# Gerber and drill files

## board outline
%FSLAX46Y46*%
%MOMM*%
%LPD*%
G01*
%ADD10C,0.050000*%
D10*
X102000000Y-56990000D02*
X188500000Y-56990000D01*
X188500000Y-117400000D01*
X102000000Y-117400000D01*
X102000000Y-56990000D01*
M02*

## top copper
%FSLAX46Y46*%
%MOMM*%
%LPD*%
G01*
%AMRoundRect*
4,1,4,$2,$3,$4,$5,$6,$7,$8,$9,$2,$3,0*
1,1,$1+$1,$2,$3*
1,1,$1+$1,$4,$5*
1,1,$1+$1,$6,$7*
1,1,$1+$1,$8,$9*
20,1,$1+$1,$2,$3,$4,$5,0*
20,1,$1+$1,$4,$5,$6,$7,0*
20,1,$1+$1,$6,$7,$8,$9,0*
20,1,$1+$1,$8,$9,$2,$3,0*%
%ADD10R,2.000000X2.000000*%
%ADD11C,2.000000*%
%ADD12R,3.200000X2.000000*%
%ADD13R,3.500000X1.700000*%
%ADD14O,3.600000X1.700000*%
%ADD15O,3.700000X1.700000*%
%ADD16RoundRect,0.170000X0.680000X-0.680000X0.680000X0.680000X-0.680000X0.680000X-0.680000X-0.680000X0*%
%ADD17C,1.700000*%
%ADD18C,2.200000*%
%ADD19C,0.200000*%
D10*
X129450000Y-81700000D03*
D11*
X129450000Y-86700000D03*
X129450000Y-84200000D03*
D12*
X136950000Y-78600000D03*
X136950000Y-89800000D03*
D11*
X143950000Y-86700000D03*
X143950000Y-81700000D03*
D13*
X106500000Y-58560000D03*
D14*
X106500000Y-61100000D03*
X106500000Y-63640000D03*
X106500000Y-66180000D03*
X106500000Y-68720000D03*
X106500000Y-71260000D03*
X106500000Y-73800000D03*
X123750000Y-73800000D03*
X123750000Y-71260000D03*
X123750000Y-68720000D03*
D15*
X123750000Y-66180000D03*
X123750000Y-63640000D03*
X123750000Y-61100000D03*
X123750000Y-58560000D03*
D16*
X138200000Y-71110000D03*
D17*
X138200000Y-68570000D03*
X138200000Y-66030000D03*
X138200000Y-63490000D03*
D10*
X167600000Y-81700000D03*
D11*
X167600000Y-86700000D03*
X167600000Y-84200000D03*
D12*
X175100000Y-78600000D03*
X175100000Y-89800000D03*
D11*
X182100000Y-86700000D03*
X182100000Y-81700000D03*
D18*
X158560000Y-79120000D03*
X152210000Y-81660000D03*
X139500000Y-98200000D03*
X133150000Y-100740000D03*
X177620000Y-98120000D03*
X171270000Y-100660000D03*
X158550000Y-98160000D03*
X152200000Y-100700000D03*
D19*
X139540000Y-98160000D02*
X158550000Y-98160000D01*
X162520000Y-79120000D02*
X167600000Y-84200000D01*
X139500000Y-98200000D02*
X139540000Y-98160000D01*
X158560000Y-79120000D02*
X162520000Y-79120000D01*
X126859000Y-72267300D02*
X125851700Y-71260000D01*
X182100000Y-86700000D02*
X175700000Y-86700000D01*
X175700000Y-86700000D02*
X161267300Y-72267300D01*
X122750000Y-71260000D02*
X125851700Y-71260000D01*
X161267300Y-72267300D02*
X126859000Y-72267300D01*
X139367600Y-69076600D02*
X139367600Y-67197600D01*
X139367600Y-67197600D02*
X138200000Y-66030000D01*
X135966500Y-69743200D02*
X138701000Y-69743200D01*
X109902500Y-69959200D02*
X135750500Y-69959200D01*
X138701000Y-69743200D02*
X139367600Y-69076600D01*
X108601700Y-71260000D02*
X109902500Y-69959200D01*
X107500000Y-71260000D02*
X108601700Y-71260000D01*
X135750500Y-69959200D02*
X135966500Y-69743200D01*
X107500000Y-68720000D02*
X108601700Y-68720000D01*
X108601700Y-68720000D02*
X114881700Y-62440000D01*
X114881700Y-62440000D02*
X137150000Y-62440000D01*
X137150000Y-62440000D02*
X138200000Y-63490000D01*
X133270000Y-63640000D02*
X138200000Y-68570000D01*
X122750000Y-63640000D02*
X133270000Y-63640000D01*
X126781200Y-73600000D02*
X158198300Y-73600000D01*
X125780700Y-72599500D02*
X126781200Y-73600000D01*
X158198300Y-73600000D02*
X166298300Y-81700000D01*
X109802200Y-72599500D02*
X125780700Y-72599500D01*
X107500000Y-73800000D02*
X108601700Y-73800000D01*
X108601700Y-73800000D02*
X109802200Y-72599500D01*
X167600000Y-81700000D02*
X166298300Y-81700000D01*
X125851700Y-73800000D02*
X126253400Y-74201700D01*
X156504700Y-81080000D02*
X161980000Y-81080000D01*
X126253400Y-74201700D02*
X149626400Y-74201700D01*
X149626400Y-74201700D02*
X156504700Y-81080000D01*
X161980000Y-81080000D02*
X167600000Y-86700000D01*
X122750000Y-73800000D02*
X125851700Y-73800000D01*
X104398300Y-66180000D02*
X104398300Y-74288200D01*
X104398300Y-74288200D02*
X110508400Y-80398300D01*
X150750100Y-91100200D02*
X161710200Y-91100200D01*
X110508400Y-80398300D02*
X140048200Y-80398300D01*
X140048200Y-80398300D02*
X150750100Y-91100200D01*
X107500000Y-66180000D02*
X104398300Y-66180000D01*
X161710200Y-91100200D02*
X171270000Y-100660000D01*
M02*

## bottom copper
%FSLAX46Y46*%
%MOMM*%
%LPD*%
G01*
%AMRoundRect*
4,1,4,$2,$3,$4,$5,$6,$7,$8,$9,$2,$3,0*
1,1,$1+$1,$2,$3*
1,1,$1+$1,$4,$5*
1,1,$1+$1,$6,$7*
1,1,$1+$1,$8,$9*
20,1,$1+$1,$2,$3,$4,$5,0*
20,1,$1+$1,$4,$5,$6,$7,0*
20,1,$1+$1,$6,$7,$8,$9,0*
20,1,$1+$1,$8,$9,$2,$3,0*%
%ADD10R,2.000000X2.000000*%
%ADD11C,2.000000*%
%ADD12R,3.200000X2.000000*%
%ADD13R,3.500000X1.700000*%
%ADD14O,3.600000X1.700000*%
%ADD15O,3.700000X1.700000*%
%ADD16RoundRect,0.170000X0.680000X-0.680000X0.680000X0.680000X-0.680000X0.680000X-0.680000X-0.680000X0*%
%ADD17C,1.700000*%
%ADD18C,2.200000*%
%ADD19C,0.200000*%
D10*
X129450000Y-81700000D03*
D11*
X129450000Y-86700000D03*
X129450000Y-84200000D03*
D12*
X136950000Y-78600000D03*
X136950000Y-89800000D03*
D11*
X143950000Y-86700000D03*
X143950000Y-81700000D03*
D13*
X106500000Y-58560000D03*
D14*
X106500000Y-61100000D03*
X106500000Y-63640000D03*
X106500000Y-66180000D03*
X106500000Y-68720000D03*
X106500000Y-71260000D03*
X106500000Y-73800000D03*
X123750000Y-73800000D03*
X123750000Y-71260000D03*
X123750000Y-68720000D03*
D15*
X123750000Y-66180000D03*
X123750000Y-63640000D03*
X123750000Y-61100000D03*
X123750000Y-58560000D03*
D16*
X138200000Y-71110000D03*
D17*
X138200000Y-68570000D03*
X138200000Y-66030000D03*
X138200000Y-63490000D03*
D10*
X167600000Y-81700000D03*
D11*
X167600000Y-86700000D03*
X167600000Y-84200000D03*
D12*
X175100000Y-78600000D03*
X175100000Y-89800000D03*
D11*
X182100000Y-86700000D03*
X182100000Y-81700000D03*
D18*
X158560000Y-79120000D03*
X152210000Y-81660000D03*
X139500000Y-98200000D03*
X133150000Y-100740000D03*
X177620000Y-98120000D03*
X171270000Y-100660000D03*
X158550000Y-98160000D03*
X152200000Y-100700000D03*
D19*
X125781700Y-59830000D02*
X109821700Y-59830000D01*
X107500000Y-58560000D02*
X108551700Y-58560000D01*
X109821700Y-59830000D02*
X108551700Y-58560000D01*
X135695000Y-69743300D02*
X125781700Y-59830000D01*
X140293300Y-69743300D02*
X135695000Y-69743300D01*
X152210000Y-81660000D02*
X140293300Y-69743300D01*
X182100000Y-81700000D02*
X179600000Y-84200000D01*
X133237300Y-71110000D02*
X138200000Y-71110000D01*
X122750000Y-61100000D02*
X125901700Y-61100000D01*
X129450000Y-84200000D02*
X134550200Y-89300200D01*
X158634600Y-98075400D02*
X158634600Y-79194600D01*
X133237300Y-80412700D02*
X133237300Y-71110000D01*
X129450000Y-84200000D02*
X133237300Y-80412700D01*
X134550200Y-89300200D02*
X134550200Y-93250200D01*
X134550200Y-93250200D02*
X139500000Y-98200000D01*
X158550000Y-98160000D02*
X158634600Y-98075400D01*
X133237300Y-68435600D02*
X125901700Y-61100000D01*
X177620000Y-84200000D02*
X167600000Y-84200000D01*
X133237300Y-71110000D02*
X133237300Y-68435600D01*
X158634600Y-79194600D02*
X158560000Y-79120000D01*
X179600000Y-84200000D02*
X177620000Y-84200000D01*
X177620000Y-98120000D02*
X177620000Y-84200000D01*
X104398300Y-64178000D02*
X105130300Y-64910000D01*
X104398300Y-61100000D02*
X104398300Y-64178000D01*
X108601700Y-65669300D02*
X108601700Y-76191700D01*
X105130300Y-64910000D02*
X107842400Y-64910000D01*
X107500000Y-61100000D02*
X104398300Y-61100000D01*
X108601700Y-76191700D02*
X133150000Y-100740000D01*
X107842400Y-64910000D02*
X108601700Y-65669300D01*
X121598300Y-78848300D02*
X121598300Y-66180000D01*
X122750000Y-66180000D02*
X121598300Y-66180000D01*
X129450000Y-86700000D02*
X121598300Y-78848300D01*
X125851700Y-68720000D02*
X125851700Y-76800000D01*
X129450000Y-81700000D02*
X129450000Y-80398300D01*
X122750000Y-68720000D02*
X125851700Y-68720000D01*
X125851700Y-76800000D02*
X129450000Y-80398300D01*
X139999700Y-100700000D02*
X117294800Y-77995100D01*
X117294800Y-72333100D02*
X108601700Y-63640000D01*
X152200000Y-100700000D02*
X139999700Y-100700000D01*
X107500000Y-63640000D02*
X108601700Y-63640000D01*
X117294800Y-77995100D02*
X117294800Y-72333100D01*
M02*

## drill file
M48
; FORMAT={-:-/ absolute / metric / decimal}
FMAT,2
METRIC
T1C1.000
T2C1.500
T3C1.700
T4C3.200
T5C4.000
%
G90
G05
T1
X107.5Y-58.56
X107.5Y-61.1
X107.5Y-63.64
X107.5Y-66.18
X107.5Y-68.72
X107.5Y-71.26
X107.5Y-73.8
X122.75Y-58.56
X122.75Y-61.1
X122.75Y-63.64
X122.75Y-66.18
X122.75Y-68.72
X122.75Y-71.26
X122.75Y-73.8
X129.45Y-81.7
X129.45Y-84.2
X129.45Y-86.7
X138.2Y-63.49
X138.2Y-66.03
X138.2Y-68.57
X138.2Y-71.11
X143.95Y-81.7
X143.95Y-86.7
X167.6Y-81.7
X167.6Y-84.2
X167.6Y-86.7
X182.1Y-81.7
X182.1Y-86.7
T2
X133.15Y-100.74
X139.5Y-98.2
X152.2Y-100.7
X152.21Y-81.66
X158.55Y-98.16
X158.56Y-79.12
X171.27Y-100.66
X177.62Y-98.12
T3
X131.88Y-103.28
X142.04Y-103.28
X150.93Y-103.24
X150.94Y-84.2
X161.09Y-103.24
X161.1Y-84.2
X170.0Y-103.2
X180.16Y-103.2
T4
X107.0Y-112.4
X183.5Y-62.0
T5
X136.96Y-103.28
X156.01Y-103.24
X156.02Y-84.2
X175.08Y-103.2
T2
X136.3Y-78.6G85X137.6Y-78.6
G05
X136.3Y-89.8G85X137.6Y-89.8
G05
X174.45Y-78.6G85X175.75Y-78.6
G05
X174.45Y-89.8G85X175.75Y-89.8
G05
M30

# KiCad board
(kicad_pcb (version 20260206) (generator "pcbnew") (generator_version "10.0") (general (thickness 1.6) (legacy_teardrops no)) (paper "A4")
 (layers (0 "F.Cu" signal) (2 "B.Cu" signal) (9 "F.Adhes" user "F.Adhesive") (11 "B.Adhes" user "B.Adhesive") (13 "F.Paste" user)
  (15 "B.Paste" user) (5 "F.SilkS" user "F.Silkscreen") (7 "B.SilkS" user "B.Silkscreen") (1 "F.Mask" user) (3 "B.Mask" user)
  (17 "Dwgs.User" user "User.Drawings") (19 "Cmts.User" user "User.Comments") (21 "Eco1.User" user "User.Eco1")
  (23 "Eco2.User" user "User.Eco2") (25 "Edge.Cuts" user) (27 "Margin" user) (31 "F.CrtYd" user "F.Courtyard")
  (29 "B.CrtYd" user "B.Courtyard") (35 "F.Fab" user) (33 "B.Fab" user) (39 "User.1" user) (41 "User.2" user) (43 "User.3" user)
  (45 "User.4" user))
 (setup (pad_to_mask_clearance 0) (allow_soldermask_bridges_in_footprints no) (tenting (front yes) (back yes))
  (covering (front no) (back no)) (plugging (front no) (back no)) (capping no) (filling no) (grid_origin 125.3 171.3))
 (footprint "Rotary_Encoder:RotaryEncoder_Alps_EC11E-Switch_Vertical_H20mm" (layer "F.Cu") (at 129.45 81.7)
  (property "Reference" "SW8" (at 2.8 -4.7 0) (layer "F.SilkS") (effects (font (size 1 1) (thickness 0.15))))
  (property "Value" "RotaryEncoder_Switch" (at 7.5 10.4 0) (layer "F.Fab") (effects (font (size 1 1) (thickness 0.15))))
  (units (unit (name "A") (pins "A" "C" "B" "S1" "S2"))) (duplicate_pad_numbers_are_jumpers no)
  (pad "A" thru_hole rect (at 0 0) (size 2 2) (drill 1) (layers "*.Cu" "*.Mask") (remove_unused_layers no) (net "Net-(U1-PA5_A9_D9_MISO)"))
  (pad "B" thru_hole circle (at 0 5) (size 2 2) (drill 1) (layers "*.Cu" "*.Mask") (remove_unused_layers no)
   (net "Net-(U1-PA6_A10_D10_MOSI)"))
  (pad "C" thru_hole circle (at 0 2.5) (size 2 2) (drill 1) (layers "*.Cu" "*.Mask") (remove_unused_layers no) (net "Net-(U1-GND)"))
  (pad "MP" thru_hole rect (at 7.5 -3.1) (size 3.2 2) (drill oval 2.8 1.5) (layers "*.Cu" "*.Mask") (remove_unused_layers no))
  (pad "MP" thru_hole rect (at 7.5 8.1) (size 3.2 2) (drill oval 2.8 1.5) (layers "*.Cu" "*.Mask") (remove_unused_layers no))
  (pad "S1" thru_hole circle (at 14.5 5) (size 2 2) (drill 1) (layers "*.Cu" "*.Mask") (remove_unused_layers no)
   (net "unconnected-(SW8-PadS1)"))
  (pad "S2" thru_hole circle (at 14.5 0) (size 2 2) (drill 1) (layers "*.Cu" "*.Mask") (remove_unused_layers no)
   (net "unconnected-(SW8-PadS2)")))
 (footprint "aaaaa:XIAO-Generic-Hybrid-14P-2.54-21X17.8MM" (layer "F.Cu") (at 115.125 66.18)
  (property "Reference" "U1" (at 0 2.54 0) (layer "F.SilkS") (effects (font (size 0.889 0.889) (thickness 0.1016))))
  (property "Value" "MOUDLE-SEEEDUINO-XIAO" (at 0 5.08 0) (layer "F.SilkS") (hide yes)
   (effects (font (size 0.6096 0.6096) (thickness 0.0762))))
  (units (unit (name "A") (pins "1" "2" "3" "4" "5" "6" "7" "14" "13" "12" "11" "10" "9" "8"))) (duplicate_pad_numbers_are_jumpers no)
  (pad "1" thru_hole rect (at -7.625 -7.62) (size 3.5 1.7) (drill 1 (offset -1 0)) (layers "*.Cu" "*.Mask") (remove_unused_layers no)
   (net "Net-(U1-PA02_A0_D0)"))
  (pad "2" thru_hole oval (at -7.625 -5.08) (size 3.6 1.7) (drill 1 (offset -1 0)) (layers "*.Cu" "*.Mask") (remove_unused_layers no)
   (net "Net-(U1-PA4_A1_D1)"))
  (pad "3" thru_hole oval (at -7.625 -2.54) (size 3.6 1.7) (drill 1 (offset -1 0)) (layers "*.Cu" "*.Mask") (remove_unused_layers no)
   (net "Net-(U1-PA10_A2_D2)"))
  (pad "4" thru_hole oval (at -7.625 0) (size 3.6 1.7) (drill 1 (offset -1 0)) (layers "*.Cu" "*.Mask") (remove_unused_layers no)
   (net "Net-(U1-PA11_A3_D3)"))
  (pad "5" thru_hole oval (at -7.625 2.54) (size 3.6 1.7) (drill 1 (offset -1 0)) (layers "*.Cu" "*.Mask") (remove_unused_layers no)
   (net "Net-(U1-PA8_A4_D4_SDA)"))
  (pad "6" thru_hole oval (at -7.625 5.08 180) (size 3.6 1.7) (drill 1 (offset 1 0)) (layers "*.Cu" "*.Mask") (remove_unused_layers no)
   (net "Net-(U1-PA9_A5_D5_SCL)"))
  (pad "7" thru_hole oval (at -7.625 7.62) (size 3.6 1.7) (drill 1 (offset -1 0)) (layers "*.Cu" "*.Mask") (remove_unused_layers no)
   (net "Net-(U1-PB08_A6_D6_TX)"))
  (pad "8" thru_hole oval (at 7.625 7.62) (size 3.6 1.7) (drill 1 (offset 1 0)) (layers "*.Cu" "*.Mask") (remove_unused_layers no)
   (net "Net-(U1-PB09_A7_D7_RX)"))
  (pad "9" thru_hole oval (at 7.625 5.08) (size 3.6 1.7) (drill 1 (offset 1 0)) (layers "*.Cu" "*.Mask") (remove_unused_layers no)
   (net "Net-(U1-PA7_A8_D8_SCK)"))
  (pad "10" thru_hole oval (at 7.625 2.54) (size 3.6 1.7) (drill 1 (offset 1 0)) (layers "*.Cu" "*.Mask") (remove_unused_layers no)
   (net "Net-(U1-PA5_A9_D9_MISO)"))
  (pad "11" thru_hole oval (at 7.625 0) (size 3.7 1.7) (drill 1 (offset 1 0)) (layers "*.Cu" "*.Mask") (remove_unused_layers no)
   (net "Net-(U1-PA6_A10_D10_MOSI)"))
  (pad "12" thru_hole oval (at 7.625 -2.54) (size 3.7 1.7) (drill 1 (offset 1 0)) (layers "*.Cu" "*.Mask") (remove_unused_layers no)
   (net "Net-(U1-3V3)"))
  (pad "13" thru_hole oval (at 7.625 -5.08) (size 3.7 1.7) (drill 1 (offset 1 0)) (layers "*.Cu" "*.Mask") (remove_unused_layers no)
   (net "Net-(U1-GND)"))
  (pad "14" thru_hole oval (at 7.625 -7.62) (size 3.7 1.7) (drill 1 (offset 1 0)) (layers "*.Cu" "*.Mask") (remove_unused_layers no)
   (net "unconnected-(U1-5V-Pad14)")))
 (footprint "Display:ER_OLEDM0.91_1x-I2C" (layer "F.Cu") (at 138.2 71.11 90)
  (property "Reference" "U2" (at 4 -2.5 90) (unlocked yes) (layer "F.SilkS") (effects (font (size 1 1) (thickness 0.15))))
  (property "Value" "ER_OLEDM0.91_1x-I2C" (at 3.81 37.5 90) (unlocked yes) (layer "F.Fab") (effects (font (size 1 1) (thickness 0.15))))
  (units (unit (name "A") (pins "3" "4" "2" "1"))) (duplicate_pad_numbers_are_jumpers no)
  (pad "1" thru_hole roundrect (at 0 0 90) (size 1.7 1.7) (drill 1) (layers "*.Cu" "*.Mask") (remove_unused_layers no)
   (roundrect_rratio 0.1) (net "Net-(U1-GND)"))
  (pad "2" thru_hole circle (at 2.54 0 90) (size 1.7 1.7) (drill 1) (layers "*.Cu" "*.Mask") (remove_unused_layers no) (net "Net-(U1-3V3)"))
  (pad "3" thru_hole circle (at 5.08 0 90) (size 1.7 1.7) (drill 1) (layers "*.Cu" "*.Mask") (remove_unused_layers no)
   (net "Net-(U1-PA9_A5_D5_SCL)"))
  (pad "4" thru_hole circle (at 7.62 0 90) (size 1.7 1.7) (drill 1) (layers "*.Cu" "*.Mask") (remove_unused_layers no)
   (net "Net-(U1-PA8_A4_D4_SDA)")))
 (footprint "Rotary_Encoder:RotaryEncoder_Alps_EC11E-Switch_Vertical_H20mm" (layer "F.Cu") (at 167.6 81.7)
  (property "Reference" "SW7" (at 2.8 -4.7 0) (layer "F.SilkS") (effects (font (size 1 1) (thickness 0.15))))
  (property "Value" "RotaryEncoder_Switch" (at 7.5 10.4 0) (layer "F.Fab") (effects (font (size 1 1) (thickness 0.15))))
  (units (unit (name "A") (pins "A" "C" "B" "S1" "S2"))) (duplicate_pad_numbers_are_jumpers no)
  (pad "A" thru_hole rect (at 0 0) (size 2 2) (drill 1) (layers "*.Cu" "*.Mask") (remove_unused_layers no) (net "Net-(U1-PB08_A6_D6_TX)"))
  (pad "B" thru_hole circle (at 0 5) (size 2 2) (drill 1) (layers "*.Cu" "*.Mask") (remove_unused_layers no) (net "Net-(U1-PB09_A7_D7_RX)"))
  (pad "C" thru_hole circle (at 0 2.5) (size 2 2) (drill 1) (layers "*.Cu" "*.Mask") (remove_unused_layers no) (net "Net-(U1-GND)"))
  (pad "MP" thru_hole rect (at 7.5 -3.1) (size 3.2 2) (drill oval 2.8 1.5) (layers "*.Cu" "*.Mask") (remove_unused_layers no))
  (pad "MP" thru_hole rect (at 7.5 8.1) (size 3.2 2) (drill oval 2.8 1.5) (layers "*.Cu" "*.Mask") (remove_unused_layers no))
  (pad "S1" thru_hole circle (at 14.5 5) (size 2 2) (drill 1) (layers "*.Cu" "*.Mask") (remove_unused_layers no)
   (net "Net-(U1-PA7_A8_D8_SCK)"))
  (pad "S2" thru_hole circle (at 14.5 0) (size 2 2) (drill 1) (layers "*.Cu" "*.Mask") (remove_unused_layers no) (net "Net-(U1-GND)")))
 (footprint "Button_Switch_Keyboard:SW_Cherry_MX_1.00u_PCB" (layer "F.Cu") (at 158.56 79.12)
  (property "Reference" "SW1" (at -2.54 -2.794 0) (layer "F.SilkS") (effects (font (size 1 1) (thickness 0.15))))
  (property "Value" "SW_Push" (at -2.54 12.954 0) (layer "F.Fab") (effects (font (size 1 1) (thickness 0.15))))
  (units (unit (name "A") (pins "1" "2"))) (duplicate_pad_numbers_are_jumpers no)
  (pad "" np_thru_hole circle (at -7.62 5.08) (size 1.7 1.7) (drill 1.7) (layers "*.Cu" "*.Mask"))
  (pad "" np_thru_hole circle (at -2.54 5.08) (size 4 4) (drill 4) (layers "*.Cu" "*.Mask"))
  (pad "" np_thru_hole circle (at 2.54 5.08) (size 1.7 1.7) (drill 1.7) (layers "*.Cu" "*.Mask"))
  (pad "1" thru_hole circle (at 0 0) (size 2.2 2.2) (drill 1.5) (layers "*.Cu" "*.Mask") (remove_unused_layers no) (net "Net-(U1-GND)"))
  (pad "2" thru_hole circle (at -6.35 2.54) (size 2.2 2.2) (drill 1.5) (layers "*.Cu" "*.Mask") (remove_unused_layers no)
   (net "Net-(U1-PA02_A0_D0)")))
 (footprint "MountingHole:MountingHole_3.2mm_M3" (layer "F.Cu") (at 183.5 62)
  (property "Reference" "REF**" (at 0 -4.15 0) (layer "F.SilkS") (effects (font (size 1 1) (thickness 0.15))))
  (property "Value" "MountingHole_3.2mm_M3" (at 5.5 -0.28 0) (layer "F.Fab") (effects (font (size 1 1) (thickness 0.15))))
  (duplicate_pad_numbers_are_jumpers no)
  (pad "" np_thru_hole circle (at 0 0) (size 3.2 3.2) (drill 3.2) (layers "*.Cu" "*.Mask")))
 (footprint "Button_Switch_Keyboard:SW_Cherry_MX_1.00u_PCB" (layer "F.Cu") (at 139.5 98.2)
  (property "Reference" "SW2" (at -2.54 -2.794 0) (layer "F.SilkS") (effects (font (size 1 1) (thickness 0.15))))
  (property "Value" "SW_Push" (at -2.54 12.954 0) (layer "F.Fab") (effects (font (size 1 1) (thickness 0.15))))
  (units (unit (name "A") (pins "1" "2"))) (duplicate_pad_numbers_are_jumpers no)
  (pad "" np_thru_hole circle (at -7.62 5.08) (size 1.7 1.7) (drill 1.7) (layers "*.Cu" "*.Mask"))
  (pad "" np_thru_hole circle (at -2.54 5.08) (size 4 4) (drill 4) (layers "*.Cu" "*.Mask"))
  (pad "" np_thru_hole circle (at 2.54 5.08) (size 1.7 1.7) (drill 1.7) (layers "*.Cu" "*.Mask"))
  (pad "1" thru_hole circle (at 0 0) (size 2.2 2.2) (drill 1.5) (layers "*.Cu" "*.Mask") (remove_unused_layers no) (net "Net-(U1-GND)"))
  (pad "2" thru_hole circle (at -6.35 2.54) (size 2.2 2.2) (drill 1.5) (layers "*.Cu" "*.Mask") (remove_unused_layers no)
   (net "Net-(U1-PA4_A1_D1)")))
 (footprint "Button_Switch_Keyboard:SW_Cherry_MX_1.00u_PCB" (layer "F.Cu") (at 177.62 98.12)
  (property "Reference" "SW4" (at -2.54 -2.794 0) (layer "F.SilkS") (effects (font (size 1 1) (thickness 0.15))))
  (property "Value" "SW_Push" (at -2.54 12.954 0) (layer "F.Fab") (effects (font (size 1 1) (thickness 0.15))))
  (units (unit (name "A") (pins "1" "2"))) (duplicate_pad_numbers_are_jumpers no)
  (pad "" np_thru_hole circle (at -7.62 5.08) (size 1.7 1.7) (drill 1.7) (layers "*.Cu" "*.Mask"))
  (pad "" np_thru_hole circle (at -2.54 5.08) (size 4 4) (drill 4) (layers "*.Cu" "*.Mask"))
  (pad "" np_thru_hole circle (at 2.54 5.08) (size 1.7 1.7) (drill 1.7) (layers "*.Cu" "*.Mask"))
  (pad "1" thru_hole circle (at 0 0) (size 2.2 2.2) (drill 1.5) (layers "*.Cu" "*.Mask") (remove_unused_layers no) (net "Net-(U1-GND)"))
  (pad "2" thru_hole circle (at -6.35 2.54) (size 2.2 2.2) (drill 1.5) (layers "*.Cu" "*.Mask") (remove_unused_layers no)
   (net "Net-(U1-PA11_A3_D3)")))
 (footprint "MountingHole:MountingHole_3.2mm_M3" (layer "F.Cu") (at 107 112.4)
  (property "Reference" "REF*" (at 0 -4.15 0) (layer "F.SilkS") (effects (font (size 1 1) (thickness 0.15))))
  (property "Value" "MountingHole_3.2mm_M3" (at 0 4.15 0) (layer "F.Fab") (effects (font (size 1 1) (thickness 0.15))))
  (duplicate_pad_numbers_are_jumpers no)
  (pad "" np_thru_hole circle (at 0 0) (size 3.2 3.2) (drill 3.2) (layers "*.Cu" "*.Mask")))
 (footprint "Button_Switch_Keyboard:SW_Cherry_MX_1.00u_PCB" (layer "F.Cu") (at 158.55 98.16)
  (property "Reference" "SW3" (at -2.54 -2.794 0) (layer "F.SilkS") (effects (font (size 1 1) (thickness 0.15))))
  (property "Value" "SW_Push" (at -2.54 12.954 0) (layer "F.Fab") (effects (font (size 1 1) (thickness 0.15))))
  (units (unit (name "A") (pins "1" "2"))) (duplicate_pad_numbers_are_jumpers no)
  (pad "" np_thru_hole circle (at -7.62 5.08) (size 1.7 1.7) (drill 1.7) (layers "*.Cu" "*.Mask"))
  (pad "" np_thru_hole circle (at -2.54 5.08) (size 4 4) (drill 4) (layers "*.Cu" "*.Mask"))
  (pad "" np_thru_hole circle (at 2.54 5.08) (size 1.7 1.7) (drill 1.7) (layers "*.Cu" "*.Mask"))
  (pad "1" thru_hole circle (at 0 0) (size 2.2 2.2) (drill 1.5) (layers "*.Cu" "*.Mask") (remove_unused_layers no) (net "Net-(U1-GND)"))
  (pad "2" thru_hole circle (at -6.35 2.54) (size 2.2 2.2) (drill 1.5) (layers "*.Cu" "*.Mask") (remove_unused_layers no)
   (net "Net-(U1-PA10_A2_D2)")))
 (gr_rect (start 102 56.99) (end 188.5 117.4) (stroke (width 0.05) (type default)) (fill no) (layer "Edge.Cuts"))
 (segment (start 125.7817 59.83) (end 109.8217 59.83) (width 0.2) (layer "B.Cu") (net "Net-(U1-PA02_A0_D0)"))
 (segment (start 107.5 58.56) (end 108.5517 58.56) (width 0.2) (layer "B.Cu") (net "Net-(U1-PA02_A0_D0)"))
 (segment (start 109.8217 59.83) (end 108.5517 58.56) (width 0.2) (layer "B.Cu") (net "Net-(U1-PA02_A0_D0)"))
 (segment (start 135.695 69.7433) (end 125.7817 59.83) (width 0.2) (layer "B.Cu") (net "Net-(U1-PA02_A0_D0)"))
 (segment (start 140.2933 69.7433) (end 135.695 69.7433) (width 0.2) (layer "B.Cu") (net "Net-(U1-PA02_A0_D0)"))
 (segment (start 152.21 81.66) (end 140.2933 69.7433) (width 0.2) (layer "B.Cu") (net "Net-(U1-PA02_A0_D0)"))
 (segment (start 139.54 98.16) (end 158.55 98.16) (width 0.2) (layer "F.Cu") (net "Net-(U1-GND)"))
 (segment (start 162.52 79.12) (end 167.6 84.2) (width 0.2) (layer "F.Cu") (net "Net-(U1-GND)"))
 (segment (start 139.5 98.2) (end 139.54 98.16) (width 0.2) (layer "F.Cu") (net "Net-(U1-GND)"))
 (segment (start 158.56 79.12) (end 162.52 79.12) (width 0.2) (layer "F.Cu") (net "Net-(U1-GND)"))
 (segment (start 182.1 81.7) (end 179.6 84.2) (width 0.2) (layer "B.Cu") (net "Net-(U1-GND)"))
 (segment (start 133.2373 71.11) (end 138.2 71.11) (width 0.2) (layer "B.Cu") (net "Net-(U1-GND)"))
 (segment (start 122.75 61.1) (end 125.9017 61.1) (width 0.2) (layer "B.Cu") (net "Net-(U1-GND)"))
 (segment (start 129.45 84.2) (end 134.5502 89.3002) (width 0.2) (layer "B.Cu") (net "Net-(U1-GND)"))
 (segment (start 158.6346 98.0754) (end 158.6346 79.1946) (width 0.2) (layer "B.Cu") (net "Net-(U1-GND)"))
 (segment (start 133.2373 80.4127) (end 133.2373 71.11) (width 0.2) (layer "B.Cu") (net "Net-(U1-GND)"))
 (segment (start 129.45 84.2) (end 133.2373 80.4127) (width 0.2) (layer "B.Cu") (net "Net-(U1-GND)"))
 (segment (start 134.5502 89.3002) (end 134.5502 93.2502) (width 0.2) (layer "B.Cu") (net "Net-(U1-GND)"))
 (segment (start 134.5502 93.2502) (end 139.5 98.2) (width 0.2) (layer "B.Cu") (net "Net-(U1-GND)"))
 (segment (start 158.55 98.16) (end 158.6346 98.0754) (width 0.2) (layer "B.Cu") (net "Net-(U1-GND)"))
 (segment (start 133.2373 68.4356) (end 125.9017 61.1) (width 0.2) (layer "B.Cu") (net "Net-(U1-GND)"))
 (segment (start 177.62 84.2) (end 167.6 84.2) (width 0.2) (layer "B.Cu") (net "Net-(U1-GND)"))
 (segment (start 133.2373 71.11) (end 133.2373 68.4356) (width 0.2) (layer "B.Cu") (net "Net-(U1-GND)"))
 (segment (start 158.6346 79.1946) (end 158.56 79.12) (width 0.2) (layer "B.Cu") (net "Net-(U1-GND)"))
 (segment (start 179.6 84.2) (end 177.62 84.2) (width 0.2) (layer "B.Cu") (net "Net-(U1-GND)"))
 (segment (start 177.62 98.12) (end 177.62 84.2) (width 0.2) (layer "B.Cu") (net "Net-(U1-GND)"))
 (segment (start 104.3983 64.178) (end 105.1303 64.91) (width 0.2) (layer "B.Cu") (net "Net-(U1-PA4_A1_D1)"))
 (segment (start 104.3983 61.1) (end 104.3983 64.178) (width 0.2) (layer "B.Cu") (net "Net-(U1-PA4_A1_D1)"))
 (segment (start 108.6017 65.6693) (end 108.6017 76.1917) (width 0.2) (layer "B.Cu") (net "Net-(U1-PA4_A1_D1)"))
 (segment (start 105.1303 64.91) (end 107.8424 64.91) (width 0.2) (layer "B.Cu") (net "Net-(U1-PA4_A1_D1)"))
 (segment (start 107.5 61.1) (end 104.3983 61.1) (width 0.2) (layer "B.Cu") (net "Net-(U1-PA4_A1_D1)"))
 (segment (start 108.6017 76.1917) (end 133.15 100.74) (width 0.2) (layer "B.Cu") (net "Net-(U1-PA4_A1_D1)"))
 (segment (start 107.8424 64.91) (end 108.6017 65.6693) (width 0.2) (layer "B.Cu") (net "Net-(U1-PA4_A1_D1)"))
 (segment (start 126.859 72.2673) (end 125.8517 71.26) (width 0.2) (layer "F.Cu") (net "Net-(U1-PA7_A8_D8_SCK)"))
 (segment (start 182.1 86.7) (end 175.7 86.7) (width 0.2) (layer "F.Cu") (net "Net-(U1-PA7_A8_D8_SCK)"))
 (segment (start 175.7 86.7) (end 161.2673 72.2673) (width 0.2) (layer "F.Cu") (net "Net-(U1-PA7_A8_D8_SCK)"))
 (segment (start 122.75 71.26) (end 125.8517 71.26) (width 0.2) (layer "F.Cu") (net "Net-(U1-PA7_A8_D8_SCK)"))
 (segment (start 161.2673 72.2673) (end 126.859 72.2673) (width 0.2) (layer "F.Cu") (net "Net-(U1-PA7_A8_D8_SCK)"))
 (segment (start 121.5983 78.8483) (end 121.5983 66.18) (width 0.2) (layer "B.Cu") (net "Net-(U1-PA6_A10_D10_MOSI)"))
 (segment (start 122.75 66.18) (end 121.5983 66.18) (width 0.2) (layer "B.Cu") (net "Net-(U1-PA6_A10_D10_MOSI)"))
 (segment (start 129.45 86.7) (end 121.5983 78.8483) (width 0.2) (layer "B.Cu") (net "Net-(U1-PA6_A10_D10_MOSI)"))
 (segment (start 139.3676 69.0766) (end 139.3676 67.1976) (width 0.2) (layer "F.Cu") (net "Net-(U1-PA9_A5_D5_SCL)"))
 (segment (start 139.3676 67.1976) (end 138.2 66.03) (width 0.2) (layer "F.Cu") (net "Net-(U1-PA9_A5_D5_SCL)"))
 (segment (start 135.9665 69.7432) (end 138.701 69.7432) (width 0.2) (layer "F.Cu") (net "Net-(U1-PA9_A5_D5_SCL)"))
 (segment (start 109.9025 69.9592) (end 135.7505 69.9592) (width 0.2) (layer "F.Cu") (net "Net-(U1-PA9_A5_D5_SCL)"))
 (segment (start 138.701 69.7432) (end 139.3676 69.0766) (width 0.2) (layer "F.Cu") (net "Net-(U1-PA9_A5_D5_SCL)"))
 (segment (start 108.6017 71.26) (end 109.9025 69.9592) (width 0.2) (layer "F.Cu") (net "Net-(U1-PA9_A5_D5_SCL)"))
 (segment (start 107.5 71.26) (end 108.6017 71.26) (width 0.2) (layer "F.Cu") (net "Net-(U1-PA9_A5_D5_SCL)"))
 (segment (start 135.7505 69.9592) (end 135.9665 69.7432) (width 0.2) (layer "F.Cu") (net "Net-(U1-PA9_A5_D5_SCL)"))
 (segment (start 107.5 68.72) (end 108.6017 68.72) (width 0.2) (layer "F.Cu") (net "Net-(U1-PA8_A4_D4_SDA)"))
 (segment (start 108.6017 68.72) (end 114.8817 62.44) (width 0.2) (layer "F.Cu") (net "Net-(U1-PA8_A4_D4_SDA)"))
 (segment (start 114.8817 62.44) (end 137.15 62.44) (width 0.2) (layer "F.Cu") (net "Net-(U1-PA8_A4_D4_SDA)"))
 (segment (start 137.15 62.44) (end 138.2 63.49) (width 0.2) (layer "F.Cu") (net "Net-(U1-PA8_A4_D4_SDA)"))
 (segment (start 133.27 63.64) (end 138.2 68.57) (width 0.2) (layer "F.Cu") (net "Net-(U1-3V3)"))
 (segment (start 122.75 63.64) (end 133.27 63.64) (width 0.2) (layer "F.Cu") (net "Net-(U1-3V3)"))
 (segment (start 126.7812 73.6) (end 158.1983 73.6) (width 0.2) (layer "F.Cu") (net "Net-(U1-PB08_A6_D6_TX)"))
 (segment (start 125.7807 72.5995) (end 126.7812 73.6) (width 0.2) (layer "F.Cu") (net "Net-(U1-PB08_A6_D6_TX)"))
 (segment (start 158.1983 73.6) (end 166.2983 81.7) (width 0.2) (layer "F.Cu") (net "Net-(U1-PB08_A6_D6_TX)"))
 (segment (start 109.8022 72.5995) (end 125.7807 72.5995) (width 0.2) (layer "F.Cu") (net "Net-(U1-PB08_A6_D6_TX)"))
 (segment (start 107.5 73.8) (end 108.6017 73.8) (width 0.2) (layer "F.Cu") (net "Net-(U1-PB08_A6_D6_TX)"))
 (segment (start 108.6017 73.8) (end 109.8022 72.5995) (width 0.2) (layer "F.Cu") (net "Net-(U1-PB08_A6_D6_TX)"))
 (segment (start 167.6 81.7) (end 166.2983 81.7) (width 0.2) (layer "F.Cu") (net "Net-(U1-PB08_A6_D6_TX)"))
 (segment (start 125.8517 73.8) (end 126.2534 74.2017) (width 0.2) (layer "F.Cu") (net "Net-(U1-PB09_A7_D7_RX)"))
 (segment (start 156.5047 81.08) (end 161.98 81.08) (width 0.2) (layer "F.Cu") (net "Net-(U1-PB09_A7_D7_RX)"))
 (segment (start 126.2534 74.2017) (end 149.6264 74.2017) (width 0.2) (layer "F.Cu") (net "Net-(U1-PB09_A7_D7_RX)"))
 (segment (start 149.6264 74.2017) (end 156.5047 81.08) (width 0.2) (layer "F.Cu") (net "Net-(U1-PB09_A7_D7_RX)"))
 (segment (start 161.98 81.08) (end 167.6 86.7) (width 0.2) (layer "F.Cu") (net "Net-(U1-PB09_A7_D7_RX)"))
 (segment (start 122.75 73.8) (end 125.8517 73.8) (width 0.2) (layer "F.Cu") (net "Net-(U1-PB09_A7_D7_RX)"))
 (segment (start 125.8517 68.72) (end 125.8517 76.8) (width 0.2) (layer "B.Cu") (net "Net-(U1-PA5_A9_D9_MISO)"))
 (segment (start 129.45 81.7) (end 129.45 80.3983) (width 0.2) (layer "B.Cu") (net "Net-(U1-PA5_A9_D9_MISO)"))
 (segment (start 122.75 68.72) (end 125.8517 68.72) (width 0.2) (layer "B.Cu") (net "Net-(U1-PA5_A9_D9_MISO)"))
 (segment (start 125.8517 76.8) (end 129.45 80.3983) (width 0.2) (layer "B.Cu") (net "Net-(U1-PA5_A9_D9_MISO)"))
 (segment (start 139.9997 100.7) (end 117.2948 77.9951) (width 0.2) (layer "B.Cu") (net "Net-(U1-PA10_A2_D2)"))
 (segment (start 117.2948 72.3331) (end 108.6017 63.64) (width 0.2) (layer "B.Cu") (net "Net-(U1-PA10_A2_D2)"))
 (segment (start 152.2 100.7) (end 139.9997 100.7) (width 0.2) (layer "B.Cu") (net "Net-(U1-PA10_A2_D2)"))
 (segment (start 107.5 63.64) (end 108.6017 63.64) (width 0.2) (layer "B.Cu") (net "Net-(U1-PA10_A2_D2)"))
 (segment (start 117.2948 77.9951) (end 117.2948 72.3331) (width 0.2) (layer "B.Cu") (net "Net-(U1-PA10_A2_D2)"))
 (segment (start 104.3983 66.18) (end 104.3983 74.2882) (width 0.2) (layer "F.Cu") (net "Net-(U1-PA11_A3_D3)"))
 (segment (start 104.3983 74.2882) (end 110.5084 80.3983) (width 0.2) (layer "F.Cu") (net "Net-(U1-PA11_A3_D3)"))
 (segment (start 150.7501 91.1002) (end 161.7102 91.1002) (width 0.2) (layer "F.Cu") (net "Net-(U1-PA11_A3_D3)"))
 (segment (start 110.5084 80.3983) (end 140.0482 80.3983) (width 0.2) (layer "F.Cu") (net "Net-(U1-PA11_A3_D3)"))
 (segment (start 140.0482 80.3983) (end 150.7501 91.1002) (width 0.2) (layer "F.Cu") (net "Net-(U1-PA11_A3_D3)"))
 (segment (start 107.5 66.18) (end 104.3983 66.18) (width 0.2) (layer "F.Cu") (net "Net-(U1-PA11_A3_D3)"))
 (segment (start 161.7102 91.1002) (end 171.27 100.66) (width 0.2) (layer "F.Cu") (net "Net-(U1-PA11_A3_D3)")))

